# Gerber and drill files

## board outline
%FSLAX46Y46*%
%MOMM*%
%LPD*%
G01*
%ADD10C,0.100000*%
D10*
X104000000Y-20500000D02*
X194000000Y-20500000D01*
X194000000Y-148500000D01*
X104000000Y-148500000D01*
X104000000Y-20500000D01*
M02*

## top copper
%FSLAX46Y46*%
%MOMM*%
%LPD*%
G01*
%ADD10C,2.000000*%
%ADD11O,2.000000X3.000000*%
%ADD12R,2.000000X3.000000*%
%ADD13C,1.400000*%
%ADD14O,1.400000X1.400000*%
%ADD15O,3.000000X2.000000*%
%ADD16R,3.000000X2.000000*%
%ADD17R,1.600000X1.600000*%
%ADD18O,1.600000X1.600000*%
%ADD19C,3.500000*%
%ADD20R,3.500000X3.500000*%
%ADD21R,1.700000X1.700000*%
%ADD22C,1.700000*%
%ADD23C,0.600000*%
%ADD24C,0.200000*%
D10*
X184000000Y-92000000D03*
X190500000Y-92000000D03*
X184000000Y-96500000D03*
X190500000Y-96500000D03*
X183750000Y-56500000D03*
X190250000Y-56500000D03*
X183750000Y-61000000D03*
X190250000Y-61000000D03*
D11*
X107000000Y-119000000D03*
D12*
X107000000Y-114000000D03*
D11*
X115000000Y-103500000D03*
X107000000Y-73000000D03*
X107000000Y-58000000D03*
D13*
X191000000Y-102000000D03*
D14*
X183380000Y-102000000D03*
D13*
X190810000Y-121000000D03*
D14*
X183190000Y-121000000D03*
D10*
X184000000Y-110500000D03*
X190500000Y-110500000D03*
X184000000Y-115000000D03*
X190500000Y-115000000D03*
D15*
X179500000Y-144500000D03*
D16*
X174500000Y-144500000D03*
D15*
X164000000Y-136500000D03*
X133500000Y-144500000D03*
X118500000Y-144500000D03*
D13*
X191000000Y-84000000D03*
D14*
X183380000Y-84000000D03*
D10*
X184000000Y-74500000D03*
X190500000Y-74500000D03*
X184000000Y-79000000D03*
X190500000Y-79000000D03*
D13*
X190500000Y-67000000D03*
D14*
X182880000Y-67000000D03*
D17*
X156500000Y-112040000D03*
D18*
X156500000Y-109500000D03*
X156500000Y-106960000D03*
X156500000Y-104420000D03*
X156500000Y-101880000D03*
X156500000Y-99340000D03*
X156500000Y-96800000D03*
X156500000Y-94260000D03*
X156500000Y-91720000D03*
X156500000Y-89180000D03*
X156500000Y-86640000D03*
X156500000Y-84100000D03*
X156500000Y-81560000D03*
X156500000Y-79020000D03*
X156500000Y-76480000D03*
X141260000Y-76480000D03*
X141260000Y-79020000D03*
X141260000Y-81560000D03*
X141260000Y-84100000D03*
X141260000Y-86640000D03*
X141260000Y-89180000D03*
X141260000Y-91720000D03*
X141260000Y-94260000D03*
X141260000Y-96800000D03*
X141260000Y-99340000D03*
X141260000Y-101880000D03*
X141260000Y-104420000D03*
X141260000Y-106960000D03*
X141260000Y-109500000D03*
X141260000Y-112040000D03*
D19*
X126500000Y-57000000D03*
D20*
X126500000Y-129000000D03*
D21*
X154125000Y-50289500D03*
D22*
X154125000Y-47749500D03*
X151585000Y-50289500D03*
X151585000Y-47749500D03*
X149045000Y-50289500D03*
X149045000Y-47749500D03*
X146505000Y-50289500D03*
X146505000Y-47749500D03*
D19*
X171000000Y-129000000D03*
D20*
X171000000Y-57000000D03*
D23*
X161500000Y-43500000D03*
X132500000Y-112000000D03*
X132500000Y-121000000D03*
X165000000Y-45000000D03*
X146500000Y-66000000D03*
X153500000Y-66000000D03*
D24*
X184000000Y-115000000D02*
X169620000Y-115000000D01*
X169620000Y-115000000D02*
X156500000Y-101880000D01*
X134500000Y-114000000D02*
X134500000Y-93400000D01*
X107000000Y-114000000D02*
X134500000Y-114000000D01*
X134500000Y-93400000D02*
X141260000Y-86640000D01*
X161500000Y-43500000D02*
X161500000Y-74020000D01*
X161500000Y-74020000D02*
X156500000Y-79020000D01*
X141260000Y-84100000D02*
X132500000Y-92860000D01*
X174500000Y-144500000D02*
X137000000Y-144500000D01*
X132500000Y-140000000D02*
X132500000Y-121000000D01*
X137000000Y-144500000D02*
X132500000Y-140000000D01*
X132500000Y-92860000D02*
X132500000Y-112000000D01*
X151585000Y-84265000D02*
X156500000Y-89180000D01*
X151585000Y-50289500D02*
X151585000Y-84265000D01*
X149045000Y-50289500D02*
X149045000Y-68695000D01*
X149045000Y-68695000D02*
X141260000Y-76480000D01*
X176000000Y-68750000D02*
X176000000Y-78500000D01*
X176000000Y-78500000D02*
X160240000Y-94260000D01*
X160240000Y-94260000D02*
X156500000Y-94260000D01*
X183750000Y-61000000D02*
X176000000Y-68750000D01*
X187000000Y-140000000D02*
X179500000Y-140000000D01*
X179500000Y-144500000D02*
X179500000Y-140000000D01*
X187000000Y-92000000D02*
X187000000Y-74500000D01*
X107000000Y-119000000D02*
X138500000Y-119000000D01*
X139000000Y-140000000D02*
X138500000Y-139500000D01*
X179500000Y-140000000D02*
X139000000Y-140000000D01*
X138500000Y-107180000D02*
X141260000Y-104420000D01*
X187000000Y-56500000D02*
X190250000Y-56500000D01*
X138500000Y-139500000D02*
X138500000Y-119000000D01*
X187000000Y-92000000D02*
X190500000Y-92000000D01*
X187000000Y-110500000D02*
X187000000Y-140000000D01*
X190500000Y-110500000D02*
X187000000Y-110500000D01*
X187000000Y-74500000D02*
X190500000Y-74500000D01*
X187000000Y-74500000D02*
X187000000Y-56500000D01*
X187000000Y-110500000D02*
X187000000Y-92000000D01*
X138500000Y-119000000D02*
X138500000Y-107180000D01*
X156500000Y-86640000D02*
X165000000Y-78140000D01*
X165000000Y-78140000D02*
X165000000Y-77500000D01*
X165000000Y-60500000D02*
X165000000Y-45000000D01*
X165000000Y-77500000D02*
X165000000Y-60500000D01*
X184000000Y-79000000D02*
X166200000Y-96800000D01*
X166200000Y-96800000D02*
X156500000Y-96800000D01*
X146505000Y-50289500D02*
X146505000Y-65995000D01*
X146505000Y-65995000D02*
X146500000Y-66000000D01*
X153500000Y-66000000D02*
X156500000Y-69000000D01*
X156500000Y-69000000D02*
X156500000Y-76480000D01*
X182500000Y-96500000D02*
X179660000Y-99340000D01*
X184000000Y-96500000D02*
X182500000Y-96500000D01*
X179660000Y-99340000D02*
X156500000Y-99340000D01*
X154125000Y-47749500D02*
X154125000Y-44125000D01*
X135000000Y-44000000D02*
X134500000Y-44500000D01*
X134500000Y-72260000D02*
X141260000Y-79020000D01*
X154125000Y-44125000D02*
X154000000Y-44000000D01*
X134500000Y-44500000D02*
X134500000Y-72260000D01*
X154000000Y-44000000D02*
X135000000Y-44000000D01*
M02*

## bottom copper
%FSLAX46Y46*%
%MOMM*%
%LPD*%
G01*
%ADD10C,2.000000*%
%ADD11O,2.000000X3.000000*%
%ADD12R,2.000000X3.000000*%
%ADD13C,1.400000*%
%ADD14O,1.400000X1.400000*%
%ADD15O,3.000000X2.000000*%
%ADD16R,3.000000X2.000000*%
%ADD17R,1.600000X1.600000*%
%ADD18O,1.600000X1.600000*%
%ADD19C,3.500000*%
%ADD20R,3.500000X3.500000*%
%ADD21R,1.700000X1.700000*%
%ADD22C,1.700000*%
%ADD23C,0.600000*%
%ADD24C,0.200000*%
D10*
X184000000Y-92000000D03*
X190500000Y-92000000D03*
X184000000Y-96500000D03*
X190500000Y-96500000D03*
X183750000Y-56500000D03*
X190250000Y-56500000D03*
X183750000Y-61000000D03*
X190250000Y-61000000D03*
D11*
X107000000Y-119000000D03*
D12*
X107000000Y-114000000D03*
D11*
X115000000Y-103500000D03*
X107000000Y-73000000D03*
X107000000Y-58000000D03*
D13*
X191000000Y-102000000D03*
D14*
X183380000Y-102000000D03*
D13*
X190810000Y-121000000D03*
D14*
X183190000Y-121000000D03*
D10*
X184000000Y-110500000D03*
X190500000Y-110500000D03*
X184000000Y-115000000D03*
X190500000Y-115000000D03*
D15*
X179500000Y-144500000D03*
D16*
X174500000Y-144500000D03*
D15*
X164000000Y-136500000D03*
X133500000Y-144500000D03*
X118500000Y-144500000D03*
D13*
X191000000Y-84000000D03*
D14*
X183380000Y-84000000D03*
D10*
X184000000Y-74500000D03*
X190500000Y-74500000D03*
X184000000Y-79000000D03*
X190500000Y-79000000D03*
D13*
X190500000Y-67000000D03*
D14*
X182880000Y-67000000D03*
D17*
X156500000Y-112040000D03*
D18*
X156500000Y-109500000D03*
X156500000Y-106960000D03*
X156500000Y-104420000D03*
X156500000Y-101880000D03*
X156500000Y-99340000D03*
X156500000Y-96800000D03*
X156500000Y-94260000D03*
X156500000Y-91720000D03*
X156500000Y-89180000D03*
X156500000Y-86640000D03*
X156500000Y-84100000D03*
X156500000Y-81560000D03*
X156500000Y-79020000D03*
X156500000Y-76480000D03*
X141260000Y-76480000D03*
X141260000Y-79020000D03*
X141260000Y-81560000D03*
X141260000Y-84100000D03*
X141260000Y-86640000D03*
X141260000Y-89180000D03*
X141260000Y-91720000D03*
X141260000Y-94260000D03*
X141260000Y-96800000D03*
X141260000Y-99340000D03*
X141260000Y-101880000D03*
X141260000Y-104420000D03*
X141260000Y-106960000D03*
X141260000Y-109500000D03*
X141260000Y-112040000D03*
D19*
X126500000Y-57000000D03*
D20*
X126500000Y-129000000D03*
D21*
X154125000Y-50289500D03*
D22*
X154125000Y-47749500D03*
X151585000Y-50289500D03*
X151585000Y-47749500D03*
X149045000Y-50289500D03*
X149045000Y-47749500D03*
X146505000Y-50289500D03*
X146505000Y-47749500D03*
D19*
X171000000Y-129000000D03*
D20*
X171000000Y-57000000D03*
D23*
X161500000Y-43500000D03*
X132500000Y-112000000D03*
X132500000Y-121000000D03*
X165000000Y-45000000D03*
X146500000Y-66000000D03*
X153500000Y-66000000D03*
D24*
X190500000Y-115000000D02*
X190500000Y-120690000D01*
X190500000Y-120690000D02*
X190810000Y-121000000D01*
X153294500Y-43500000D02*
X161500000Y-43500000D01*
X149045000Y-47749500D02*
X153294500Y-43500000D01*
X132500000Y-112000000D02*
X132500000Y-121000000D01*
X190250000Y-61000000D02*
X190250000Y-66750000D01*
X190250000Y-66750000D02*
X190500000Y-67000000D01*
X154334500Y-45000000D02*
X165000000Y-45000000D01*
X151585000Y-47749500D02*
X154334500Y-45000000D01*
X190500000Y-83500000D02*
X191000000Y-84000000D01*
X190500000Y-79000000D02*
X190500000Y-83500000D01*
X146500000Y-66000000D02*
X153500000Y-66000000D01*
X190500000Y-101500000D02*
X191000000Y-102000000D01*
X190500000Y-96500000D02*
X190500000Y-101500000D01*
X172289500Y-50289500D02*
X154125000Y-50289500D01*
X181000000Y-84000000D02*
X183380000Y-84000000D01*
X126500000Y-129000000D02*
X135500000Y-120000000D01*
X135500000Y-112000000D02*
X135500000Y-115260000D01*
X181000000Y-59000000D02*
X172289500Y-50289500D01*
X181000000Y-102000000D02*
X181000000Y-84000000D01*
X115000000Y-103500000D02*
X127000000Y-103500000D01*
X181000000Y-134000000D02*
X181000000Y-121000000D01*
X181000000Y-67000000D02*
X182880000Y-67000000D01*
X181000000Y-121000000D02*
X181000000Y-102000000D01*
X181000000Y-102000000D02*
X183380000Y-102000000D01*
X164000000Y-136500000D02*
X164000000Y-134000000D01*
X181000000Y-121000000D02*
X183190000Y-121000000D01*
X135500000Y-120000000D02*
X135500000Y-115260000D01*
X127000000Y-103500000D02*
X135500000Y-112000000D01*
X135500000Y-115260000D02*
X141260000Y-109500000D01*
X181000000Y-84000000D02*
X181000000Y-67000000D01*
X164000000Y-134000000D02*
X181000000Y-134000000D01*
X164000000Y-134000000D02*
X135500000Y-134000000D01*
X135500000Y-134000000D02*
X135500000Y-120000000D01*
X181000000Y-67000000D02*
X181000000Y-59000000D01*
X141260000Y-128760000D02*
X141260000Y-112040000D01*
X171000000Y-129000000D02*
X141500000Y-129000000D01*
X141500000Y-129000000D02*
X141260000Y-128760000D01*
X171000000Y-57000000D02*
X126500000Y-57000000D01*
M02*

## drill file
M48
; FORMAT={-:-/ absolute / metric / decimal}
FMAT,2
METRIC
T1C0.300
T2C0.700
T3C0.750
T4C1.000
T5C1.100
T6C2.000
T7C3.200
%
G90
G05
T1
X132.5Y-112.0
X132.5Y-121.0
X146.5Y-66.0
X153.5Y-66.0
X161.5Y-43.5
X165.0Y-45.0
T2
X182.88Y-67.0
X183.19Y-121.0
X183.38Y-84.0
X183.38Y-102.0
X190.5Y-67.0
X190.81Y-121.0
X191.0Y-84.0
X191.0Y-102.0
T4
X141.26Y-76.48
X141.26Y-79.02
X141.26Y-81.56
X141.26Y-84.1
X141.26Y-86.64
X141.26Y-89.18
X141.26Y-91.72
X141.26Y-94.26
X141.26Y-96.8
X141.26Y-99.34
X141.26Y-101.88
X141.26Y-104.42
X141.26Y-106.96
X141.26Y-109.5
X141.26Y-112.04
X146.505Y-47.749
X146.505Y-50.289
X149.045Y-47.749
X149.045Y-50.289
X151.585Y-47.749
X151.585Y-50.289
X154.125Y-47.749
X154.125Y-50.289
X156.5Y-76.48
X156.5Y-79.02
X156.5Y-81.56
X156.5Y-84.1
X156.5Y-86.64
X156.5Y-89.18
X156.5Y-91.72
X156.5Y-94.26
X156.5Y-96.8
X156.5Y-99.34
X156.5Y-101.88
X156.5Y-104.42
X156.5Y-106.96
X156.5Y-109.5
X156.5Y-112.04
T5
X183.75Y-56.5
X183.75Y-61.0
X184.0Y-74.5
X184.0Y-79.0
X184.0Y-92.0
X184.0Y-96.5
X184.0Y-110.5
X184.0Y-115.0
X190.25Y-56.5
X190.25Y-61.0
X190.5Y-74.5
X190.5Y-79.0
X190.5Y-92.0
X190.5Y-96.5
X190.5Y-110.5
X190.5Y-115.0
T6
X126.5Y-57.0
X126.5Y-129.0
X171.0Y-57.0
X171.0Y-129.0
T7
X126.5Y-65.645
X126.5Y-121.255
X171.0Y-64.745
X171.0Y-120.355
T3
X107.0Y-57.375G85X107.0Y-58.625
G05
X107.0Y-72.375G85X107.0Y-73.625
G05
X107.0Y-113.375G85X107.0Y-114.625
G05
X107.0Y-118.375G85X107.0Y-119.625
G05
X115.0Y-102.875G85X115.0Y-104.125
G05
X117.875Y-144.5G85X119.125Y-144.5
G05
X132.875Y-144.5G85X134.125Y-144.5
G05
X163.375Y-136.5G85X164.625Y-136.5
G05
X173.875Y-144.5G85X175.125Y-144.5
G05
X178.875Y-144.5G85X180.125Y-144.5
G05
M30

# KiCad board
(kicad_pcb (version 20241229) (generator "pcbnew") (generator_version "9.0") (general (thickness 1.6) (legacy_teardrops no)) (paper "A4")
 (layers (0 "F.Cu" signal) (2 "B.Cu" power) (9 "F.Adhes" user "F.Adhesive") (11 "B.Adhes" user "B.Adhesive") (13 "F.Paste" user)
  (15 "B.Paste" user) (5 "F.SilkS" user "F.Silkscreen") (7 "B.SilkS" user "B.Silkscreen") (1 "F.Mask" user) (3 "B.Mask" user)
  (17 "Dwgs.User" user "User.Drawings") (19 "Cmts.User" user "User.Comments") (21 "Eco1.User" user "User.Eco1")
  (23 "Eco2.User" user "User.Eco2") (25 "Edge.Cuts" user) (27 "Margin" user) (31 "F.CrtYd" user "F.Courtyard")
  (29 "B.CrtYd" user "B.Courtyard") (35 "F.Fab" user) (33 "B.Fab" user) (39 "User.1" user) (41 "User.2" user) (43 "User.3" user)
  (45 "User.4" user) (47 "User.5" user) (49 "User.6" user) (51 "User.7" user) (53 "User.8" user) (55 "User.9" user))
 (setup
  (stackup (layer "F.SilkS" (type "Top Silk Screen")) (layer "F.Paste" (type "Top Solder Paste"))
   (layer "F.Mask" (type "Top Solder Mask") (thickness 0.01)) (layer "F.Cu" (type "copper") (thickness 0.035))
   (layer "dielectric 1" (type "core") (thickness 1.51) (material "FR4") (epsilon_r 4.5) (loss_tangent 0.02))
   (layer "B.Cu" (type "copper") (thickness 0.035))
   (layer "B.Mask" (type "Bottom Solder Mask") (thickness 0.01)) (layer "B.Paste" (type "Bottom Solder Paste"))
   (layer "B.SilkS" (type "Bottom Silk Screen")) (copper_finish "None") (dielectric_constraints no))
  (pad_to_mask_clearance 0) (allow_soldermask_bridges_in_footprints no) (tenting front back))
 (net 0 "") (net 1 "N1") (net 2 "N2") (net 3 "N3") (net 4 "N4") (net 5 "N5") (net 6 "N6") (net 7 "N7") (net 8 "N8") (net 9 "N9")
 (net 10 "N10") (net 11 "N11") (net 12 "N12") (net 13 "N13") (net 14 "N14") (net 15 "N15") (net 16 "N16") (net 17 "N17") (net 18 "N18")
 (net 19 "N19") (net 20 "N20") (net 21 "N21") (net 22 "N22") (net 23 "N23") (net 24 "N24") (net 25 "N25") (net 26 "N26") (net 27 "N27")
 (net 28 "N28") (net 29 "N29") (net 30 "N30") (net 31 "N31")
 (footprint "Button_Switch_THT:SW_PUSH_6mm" (layer "F.Cu") (at 184 92)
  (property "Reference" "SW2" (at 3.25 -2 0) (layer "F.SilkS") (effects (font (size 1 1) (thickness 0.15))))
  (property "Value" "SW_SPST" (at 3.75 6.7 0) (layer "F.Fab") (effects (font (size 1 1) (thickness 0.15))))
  (pad "1" thru_hole circle (at 0 0 90) (size 2 2) (drill 1.1) (layers "*.Cu" "*.Mask") (remove_unused_layers no) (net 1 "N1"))
  (pad "1" thru_hole circle (at 6.5 0 90) (size 2 2) (drill 1.1) (layers "*.Cu" "*.Mask") (remove_unused_layers no) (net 1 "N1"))
  (pad "2" thru_hole circle (at 0 4.5 90) (size 2 2) (drill 1.1) (layers "*.Cu" "*.Mask") (remove_unused_layers no) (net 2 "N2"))
  (pad "2" thru_hole circle (at 6.5 4.5 90) (size 2 2) (drill 1.1) (layers "*.Cu" "*.Mask") (remove_unused_layers no) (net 2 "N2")))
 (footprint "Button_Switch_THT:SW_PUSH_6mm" (layer "F.Cu") (at 183.75 56.5)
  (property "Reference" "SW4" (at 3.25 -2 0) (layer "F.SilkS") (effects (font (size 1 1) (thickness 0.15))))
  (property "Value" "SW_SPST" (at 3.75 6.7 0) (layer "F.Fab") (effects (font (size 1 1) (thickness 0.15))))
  (pad "1" thru_hole circle (at 0 0 90) (size 2 2) (drill 1.1) (layers "*.Cu" "*.Mask") (remove_unused_layers no) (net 1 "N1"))
  (pad "1" thru_hole circle (at 6.5 0 90) (size 2 2) (drill 1.1) (layers "*.Cu" "*.Mask") (remove_unused_layers no) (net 1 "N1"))
  (pad "2" thru_hole circle (at 0 4.5 90) (size 2 2) (drill 1.1) (layers "*.Cu" "*.Mask") (remove_unused_layers no) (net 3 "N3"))
  (pad "2" thru_hole circle (at 6.5 4.5 90) (size 2 2) (drill 1.1) (layers "*.Cu" "*.Mask") (remove_unused_layers no) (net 3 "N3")))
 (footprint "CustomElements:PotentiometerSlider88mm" (layer "F.Cu") (at 111 88.5 -90)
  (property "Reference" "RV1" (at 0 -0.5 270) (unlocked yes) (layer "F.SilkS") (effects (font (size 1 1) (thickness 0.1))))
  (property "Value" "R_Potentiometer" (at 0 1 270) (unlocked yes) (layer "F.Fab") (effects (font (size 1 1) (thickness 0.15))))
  (pad "1" thru_hole oval (at 30.5 4 270) (size 3 2) (drill oval 2 0.75) (layers "*.Cu" "*.Mask") (remove_unused_layers no) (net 1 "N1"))
  (pad "2" thru_hole rect (at 25.5 4 270) (size 3 2) (drill oval 2 0.75) (layers "*.Cu" "*.Mask") (remove_unused_layers no) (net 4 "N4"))
  (pad "3" thru_hole oval (at 15 -4 270) (size 3 2) (drill oval 2 0.75) (layers "*.Cu" "*.Mask") (remove_unused_layers no) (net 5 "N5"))
  (pad "4" thru_hole oval (at -15.5 4 270) (size 3 2) (drill oval 2 0.75) (layers "*.Cu" "*.Mask") (remove_unused_layers no))
  (pad "5" thru_hole oval (at -30.5 4 270) (size 3 2) (drill oval 2 0.75) (layers "*.Cu" "*.Mask") (remove_unused_layers no)))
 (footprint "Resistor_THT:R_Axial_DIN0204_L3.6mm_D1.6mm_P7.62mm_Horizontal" (layer "F.Cu") (at 191 102 180)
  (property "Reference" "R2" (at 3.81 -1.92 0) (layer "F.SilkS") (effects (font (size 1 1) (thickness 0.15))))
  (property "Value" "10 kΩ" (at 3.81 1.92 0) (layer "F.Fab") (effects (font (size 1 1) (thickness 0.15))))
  (pad "1" thru_hole circle (at 0 0 180) (size 1.4 1.4) (drill 0.7) (layers "*.Cu" "*.Mask") (remove_unused_layers no) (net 2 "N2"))
  (pad "2" thru_hole oval (at 7.62 0 180) (size 1.4 1.4) (drill 0.7) (layers "*.Cu" "*.Mask") (remove_unused_layers no) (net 5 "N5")))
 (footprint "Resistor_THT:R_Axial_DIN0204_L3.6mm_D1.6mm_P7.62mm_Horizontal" (layer "F.Cu") (at 190.81 121 180)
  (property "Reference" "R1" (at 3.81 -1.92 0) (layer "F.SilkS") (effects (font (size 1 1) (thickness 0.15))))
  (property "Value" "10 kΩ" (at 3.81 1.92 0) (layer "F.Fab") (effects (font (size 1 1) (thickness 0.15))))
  (pad "1" thru_hole circle (at 0 0 180) (size 1.4 1.4) (drill 0.7) (layers "*.Cu" "*.Mask") (remove_unused_layers no) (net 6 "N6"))
  (pad "2" thru_hole oval (at 7.62 0 180) (size 1.4 1.4) (drill 0.7) (layers "*.Cu" "*.Mask") (remove_unused_layers no) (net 5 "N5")))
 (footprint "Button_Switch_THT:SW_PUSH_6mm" (layer "F.Cu") (at 184 110.5)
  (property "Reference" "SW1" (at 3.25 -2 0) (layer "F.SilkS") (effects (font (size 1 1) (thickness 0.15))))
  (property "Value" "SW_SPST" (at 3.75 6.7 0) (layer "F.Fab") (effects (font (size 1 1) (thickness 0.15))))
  (pad "1" thru_hole circle (at 0 0 90) (size 2 2) (drill 1.1) (layers "*.Cu" "*.Mask") (remove_unused_layers no) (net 1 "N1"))
  (pad "1" thru_hole circle (at 6.5 0 90) (size 2 2) (drill 1.1) (layers "*.Cu" "*.Mask") (remove_unused_layers no) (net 1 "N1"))
  (pad "2" thru_hole circle (at 0 4.5 90) (size 2 2) (drill 1.1) (layers "*.Cu" "*.Mask") (remove_unused_layers no) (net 6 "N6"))
  (pad "2" thru_hole circle (at 6.5 4.5 90) (size 2 2) (drill 1.1) (layers "*.Cu" "*.Mask") (remove_unused_layers no) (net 6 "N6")))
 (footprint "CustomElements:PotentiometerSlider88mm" (layer "F.Cu") (at 149 140.5)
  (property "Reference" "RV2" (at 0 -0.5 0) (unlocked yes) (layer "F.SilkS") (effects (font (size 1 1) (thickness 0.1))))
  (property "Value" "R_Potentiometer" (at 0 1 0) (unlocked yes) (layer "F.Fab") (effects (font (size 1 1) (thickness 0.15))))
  (pad "1" thru_hole oval (at 30.5 4) (size 3 2) (drill oval 2 0.75) (layers "*.Cu" "*.Mask") (remove_unused_layers no) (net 1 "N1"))
  (pad "2" thru_hole rect (at 25.5 4) (size 3 2) (drill oval 2 0.75) (layers "*.Cu" "*.Mask") (remove_unused_layers no) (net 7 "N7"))
  (pad "3" thru_hole oval (at 15 -4) (size 3 2) (drill oval 2 0.75) (layers "*.Cu" "*.Mask") (remove_unused_layers no) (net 5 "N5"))
  (pad "4" thru_hole oval (at -15.5 4) (size 3 2) (drill oval 2 0.75) (layers "*.Cu" "*.Mask") (remove_unused_layers no))
  (pad "5" thru_hole oval (at -30.5 4) (size 3 2) (drill oval 2 0.75) (layers "*.Cu" "*.Mask") (remove_unused_layers no)))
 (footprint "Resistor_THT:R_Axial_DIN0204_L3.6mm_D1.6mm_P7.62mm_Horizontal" (layer "F.Cu") (at 191 84 180)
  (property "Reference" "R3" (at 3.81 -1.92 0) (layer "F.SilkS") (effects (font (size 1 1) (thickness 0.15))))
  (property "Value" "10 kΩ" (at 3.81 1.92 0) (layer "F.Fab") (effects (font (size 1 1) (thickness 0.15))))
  (pad "1" thru_hole circle (at 0 0 180) (size 1.4 1.4) (drill 0.7) (layers "*.Cu" "*.Mask") (remove_unused_layers no) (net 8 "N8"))
  (pad "2" thru_hole oval (at 7.62 0 180) (size 1.4 1.4) (drill 0.7) (layers "*.Cu" "*.Mask") (remove_unused_layers no) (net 5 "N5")))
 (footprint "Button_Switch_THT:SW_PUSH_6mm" (layer "F.Cu") (at 184 74.5)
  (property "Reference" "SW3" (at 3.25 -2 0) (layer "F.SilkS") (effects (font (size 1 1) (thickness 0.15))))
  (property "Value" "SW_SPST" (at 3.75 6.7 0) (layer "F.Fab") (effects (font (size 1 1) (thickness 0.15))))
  (pad "1" thru_hole circle (at 0 0 90) (size 2 2) (drill 1.1) (layers "*.Cu" "*.Mask") (remove_unused_layers no) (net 1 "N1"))
  (pad "1" thru_hole circle (at 6.5 0 90) (size 2 2) (drill 1.1) (layers "*.Cu" "*.Mask") (remove_unused_layers no) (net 1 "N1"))
  (pad "2" thru_hole circle (at 0 4.5 90) (size 2 2) (drill 1.1) (layers "*.Cu" "*.Mask") (remove_unused_layers no) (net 8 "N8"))
  (pad "2" thru_hole circle (at 6.5 4.5 90) (size 2 2) (drill 1.1) (layers "*.Cu" "*.Mask") (remove_unused_layers no) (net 8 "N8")))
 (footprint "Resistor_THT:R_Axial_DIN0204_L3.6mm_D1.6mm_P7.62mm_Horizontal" (layer "F.Cu") (at 190.5 67 180)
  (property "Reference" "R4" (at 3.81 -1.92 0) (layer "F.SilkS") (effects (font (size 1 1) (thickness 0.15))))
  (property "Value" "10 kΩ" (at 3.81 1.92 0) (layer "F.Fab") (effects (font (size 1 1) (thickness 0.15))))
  (pad "1" thru_hole circle (at 0 0 180) (size 1.4 1.4) (drill 0.7) (layers "*.Cu" "*.Mask") (remove_unused_layers no) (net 3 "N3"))
  (pad "2" thru_hole oval (at 7.62 0 180) (size 1.4 1.4) (drill 0.7) (layers "*.Cu" "*.Mask") (remove_unused_layers no) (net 5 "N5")))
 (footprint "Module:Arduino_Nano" (layer "F.Cu") (at 156.5 112.04 180)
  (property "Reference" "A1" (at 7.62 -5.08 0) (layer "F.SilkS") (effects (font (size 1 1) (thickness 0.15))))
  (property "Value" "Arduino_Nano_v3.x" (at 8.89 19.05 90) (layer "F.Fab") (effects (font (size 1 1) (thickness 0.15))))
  (pad "1" thru_hole rect (at 0 0 180) (size 1.6 1.6) (drill 1) (layers "*.Cu" "*.Mask") (remove_unused_layers no) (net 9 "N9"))
  (pad "2" thru_hole oval (at 0 2.54 180) (size 1.6 1.6) (drill 1) (layers "*.Cu" "*.Mask") (remove_unused_layers no) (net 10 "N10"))
  (pad "3" thru_hole oval (at 0 5.08 180) (size 1.6 1.6) (drill 1) (layers "*.Cu" "*.Mask") (remove_unused_layers no) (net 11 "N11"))
  (pad "4" thru_hole oval (at 0 7.62 180) (size 1.6 1.6) (drill 1) (layers "*.Cu" "*.Mask") (remove_unused_layers no) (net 5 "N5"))
  (pad "5" thru_hole oval (at 0 10.16 180) (size 1.6 1.6) (drill 1) (layers "*.Cu" "*.Mask") (remove_unused_layers no) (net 6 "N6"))
  (pad "6" thru_hole oval (at 0 12.7 180) (size 1.6 1.6) (drill 1) (layers "*.Cu" "*.Mask") (remove_unused_layers no) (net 2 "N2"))
  (pad "7" thru_hole oval (at 0 15.24 180) (size 1.6 1.6) (drill 1) (layers "*.Cu" "*.Mask") (remove_unused_layers no) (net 8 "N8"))
  (pad "8" thru_hole oval (at 0 17.78 180) (size 1.6 1.6) (drill 1) (layers "*.Cu" "*.Mask") (remove_unused_layers no) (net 3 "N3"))
  (pad "9" thru_hole oval (at 0 20.32 180) (size 1.6 1.6) (drill 1) (layers "*.Cu" "*.Mask") (remove_unused_layers no) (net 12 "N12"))
  (pad "10" thru_hole oval (at 0 22.86 180) (size 1.6 1.6) (drill 1) (layers "*.Cu" "*.Mask") (remove_unused_layers no) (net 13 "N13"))
  (pad "11" thru_hole oval (at 0 25.4 180) (size 1.6 1.6) (drill 1) (layers "*.Cu" "*.Mask") (remove_unused_layers no) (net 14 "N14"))
  (pad "12" thru_hole oval (at 0 27.94 180) (size 1.6 1.6) (drill 1) (layers "*.Cu" "*.Mask") (remove_unused_layers no) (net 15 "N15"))
  (pad "13" thru_hole oval (at 0 30.48 180) (size 1.6 1.6) (drill 1) (layers "*.Cu" "*.Mask") (remove_unused_layers no) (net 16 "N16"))
  (pad "14" thru_hole oval (at 0 33.02 180) (size 1.6 1.6) (drill 1) (layers "*.Cu" "*.Mask") (remove_unused_layers no) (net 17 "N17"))
  (pad "15" thru_hole oval (at 0 35.56 180) (size 1.6 1.6) (drill 1) (layers "*.Cu" "*.Mask") (remove_unused_layers no) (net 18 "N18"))
  (pad "16" thru_hole oval (at 15.24 35.56 180) (size 1.6 1.6) (drill 1) (layers "*.Cu" "*.Mask") (remove_unused_layers no) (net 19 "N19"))
  (pad "17" thru_hole oval (at 15.24 33.02 180) (size 1.6 1.6) (drill 1) (layers "*.Cu" "*.Mask") (remove_unused_layers no) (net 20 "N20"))
  (pad "18" thru_hole oval (at 15.24 30.48 180) (size 1.6 1.6) (drill 1) (layers "*.Cu" "*.Mask") (remove_unused_layers no) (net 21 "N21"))
  (pad "19" thru_hole oval (at 15.24 27.94 180) (size 1.6 1.6) (drill 1) (layers "*.Cu" "*.Mask") (remove_unused_layers no) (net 7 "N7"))
  (pad "20" thru_hole oval (at 15.24 25.4 180) (size 1.6 1.6) (drill 1) (layers "*.Cu" "*.Mask") (remove_unused_layers no) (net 4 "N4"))
  (pad "21" thru_hole oval (at 15.24 22.86 180) (size 1.6 1.6) (drill 1) (layers "*.Cu" "*.Mask") (remove_unused_layers no) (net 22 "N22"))
  (pad "22" thru_hole oval (at 15.24 20.32 180) (size 1.6 1.6) (drill 1) (layers "*.Cu" "*.Mask") (remove_unused_layers no) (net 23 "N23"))
  (pad "23" thru_hole oval (at 15.24 17.78 180) (size 1.6 1.6) (drill 1) (layers "*.Cu" "*.Mask") (remove_unused_layers no) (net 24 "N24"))
  (pad "24" thru_hole oval (at 15.24 15.24 180) (size 1.6 1.6) (drill 1) (layers "*.Cu" "*.Mask") (remove_unused_layers no) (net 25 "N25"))
  (pad "25" thru_hole oval (at 15.24 12.7 180) (size 1.6 1.6) (drill 1) (layers "*.Cu" "*.Mask") (remove_unused_layers no) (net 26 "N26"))
  (pad "26" thru_hole oval (at 15.24 10.16 180) (size 1.6 1.6) (drill 1) (layers "*.Cu" "*.Mask") (remove_unused_layers no) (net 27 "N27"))
  (pad "27" thru_hole oval (at 15.24 7.62 180) (size 1.6 1.6) (drill 1) (layers "*.Cu" "*.Mask") (remove_unused_layers no) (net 1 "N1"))
  (pad "28" thru_hole oval (at 15.24 5.08 180) (size 1.6 1.6) (drill 1) (layers "*.Cu" "*.Mask") (remove_unused_layers no) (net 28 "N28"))
  (pad "29" thru_hole oval (at 15.24 2.54 180) (size 1.6 1.6) (drill 1) (layers "*.Cu" "*.Mask") (remove_unused_layers no) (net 5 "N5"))
  (pad "30" thru_hole oval (at 15.24 0 180) (size 1.6 1.6) (drill 1) (layers "*.Cu" "*.Mask") (remove_unused_layers no) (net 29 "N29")))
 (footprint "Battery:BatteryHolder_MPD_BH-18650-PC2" (layer "B.Cu") (at 126.5 57 -90)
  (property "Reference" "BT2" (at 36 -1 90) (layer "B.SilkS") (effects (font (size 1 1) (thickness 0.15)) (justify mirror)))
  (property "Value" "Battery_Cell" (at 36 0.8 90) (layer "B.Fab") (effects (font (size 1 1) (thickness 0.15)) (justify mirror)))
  (pad "" np_thru_hole circle (at 8.645 0 270) (size 3.2 3.2) (drill 3.2) (layers "*.Cu" "*.Mask"))
  (pad "" np_thru_hole circle (at 64.255 0 270) (size 3.2 3.2) (drill 3.2) (layers "*.Cu" "*.Mask"))
  (pad "1" thru_hole circle (at 0 0 270) (size 3.5 3.5) (drill 2) (layers "*.Cu" "*.Mask") (remove_unused_layers no) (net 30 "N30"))
  (pad "2" thru_hole rect (at 72 0 270) (size 3.5 3.5) (drill 2) (layers "*.Cu" "*.Mask") (remove_unused_layers no) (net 5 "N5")))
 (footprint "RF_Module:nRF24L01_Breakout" (layer "B.Cu") (at 154.125 50.2895 90)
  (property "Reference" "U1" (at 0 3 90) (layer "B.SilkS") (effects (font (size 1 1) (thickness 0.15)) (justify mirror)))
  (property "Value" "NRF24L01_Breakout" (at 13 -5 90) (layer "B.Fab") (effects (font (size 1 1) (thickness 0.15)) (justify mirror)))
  (pad "1" thru_hole rect (at 0 0 90) (size 1.7 1.7) (drill 1) (layers "*.Cu" "*.Mask") (remove_unused_layers no) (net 5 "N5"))
  (pad "2" thru_hole circle (at 2.54 0 90) (size 1.7 1.7) (drill 1) (layers "*.Cu" "*.Mask") (remove_unused_layers no) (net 20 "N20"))
  (pad "3" thru_hole circle (at 0 -2.54 90) (size 1.7 1.7) (drill 1) (layers "*.Cu" "*.Mask") (remove_unused_layers no) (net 13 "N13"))
  (pad "4" thru_hole circle (at 2.54 -2.54 90) (size 1.7 1.7) (drill 1) (layers "*.Cu" "*.Mask") (remove_unused_layers no) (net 14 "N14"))
  (pad "5" thru_hole circle (at 0 -5.08 90) (size 1.7 1.7) (drill 1) (layers "*.Cu" "*.Mask") (remove_unused_layers no) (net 19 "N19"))
  (pad "6" thru_hole circle (at 2.54 -5.08 90) (size 1.7 1.7) (drill 1) (layers "*.Cu" "*.Mask") (remove_unused_layers no) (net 17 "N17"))
  (pad "7" thru_hole circle (at 0 -7.62 90) (size 1.7 1.7) (drill 1) (layers "*.Cu" "*.Mask") (remove_unused_layers no) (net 18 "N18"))
  (pad "8" thru_hole circle (at 2.54 -7.62 90) (size 1.7 1.7) (drill 1) (layers "*.Cu" "*.Mask") (remove_unused_layers no) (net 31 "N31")))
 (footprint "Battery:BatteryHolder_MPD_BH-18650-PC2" (layer "B.Cu") (at 171 129 90)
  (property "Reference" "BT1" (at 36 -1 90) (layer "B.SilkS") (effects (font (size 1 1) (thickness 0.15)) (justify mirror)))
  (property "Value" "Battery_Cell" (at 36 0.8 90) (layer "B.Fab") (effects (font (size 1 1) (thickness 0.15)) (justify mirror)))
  (pad "" np_thru_hole circle (at 8.645 0 90) (size 3.2 3.2) (drill 3.2) (layers "*.Cu" "*.Mask"))
  (pad "" np_thru_hole circle (at 64.255 0 90) (size 3.2 3.2) (drill 3.2) (layers "*.Cu" "*.Mask"))
  (pad "1" thru_hole circle (at 0 0 90) (size 3.5 3.5) (drill 2) (layers "*.Cu" "*.Mask") (remove_unused_layers no) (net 29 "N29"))
  (pad "2" thru_hole rect (at 72 0 90) (size 3.5 3.5) (drill 2) (layers "*.Cu" "*.Mask") (remove_unused_layers no) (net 30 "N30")))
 (gr_rect (start 104 20.5) (end 194 148.5) (stroke (width 0.1) (type default)) (fill no) (layer "Edge.Cuts"))
 (segment (start 184 115) (end 169.62 115) (width 0.2) (layer "F.Cu") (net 6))
 (segment (start 169.62 115) (end 156.5 101.88) (width 0.2) (layer "F.Cu") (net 6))
 (segment (start 190.5 115) (end 190.5 120.69) (width 0.2) (layer "B.Cu") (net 6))
 (segment (start 190.5 120.69) (end 190.81 121) (width 0.2) (layer "B.Cu") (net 6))
 (segment (start 134.5 114) (end 134.5 93.4) (width 0.2) (layer "F.Cu") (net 4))
 (segment (start 107 114) (end 134.5 114) (width 0.2) (layer "F.Cu") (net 4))
 (segment (start 134.5 93.4) (end 141.26 86.64) (width 0.2) (layer "F.Cu") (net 4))
 (segment (start 161.5 43.5) (end 161.5 74.02) (width 0.2) (layer "F.Cu") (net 17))
 (segment (start 161.5 74.02) (end 156.5 79.02) (width 0.2) (layer "F.Cu") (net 17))
 (via (at 161.5 43.5) (size 0.6) (drill 0.3) (layers "F.Cu" "B.Cu") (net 17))
 (segment (start 153.2945 43.5) (end 161.5 43.5) (width 0.2) (layer "B.Cu") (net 17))
 (segment (start 149.045 47.7495) (end 153.2945 43.5) (width 0.2) (layer "B.Cu") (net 17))
 (segment (start 141.26 84.1) (end 132.5 92.86) (width 0.2) (layer "F.Cu") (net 7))
 (segment (start 174.5 144.5) (end 137 144.5) (width 0.2) (layer "F.Cu") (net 7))
 (segment (start 132.5 140) (end 132.5 121) (width 0.2) (layer "F.Cu") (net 7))
 (segment (start 137 144.5) (end 132.5 140) (width 0.2) (layer "F.Cu") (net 7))
 (segment (start 132.5 92.86) (end 132.5 112) (width 0.2) (layer "F.Cu") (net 7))
 (via (at 132.5 112) (size 0.6) (drill 0.3) (layers "F.Cu" "B.Cu") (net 7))
 (via (at 132.5 121) (size 0.6) (drill 0.3) (layers "F.Cu" "B.Cu") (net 7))
 (segment (start 132.5 112) (end 132.5 121) (width 0.2) (layer "B.Cu") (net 7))
 (segment (start 151.585 84.265) (end 156.5 89.18) (width 0.2) (layer "F.Cu") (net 13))
 (segment (start 151.585 50.2895) (end 151.585 84.265) (width 0.2) (layer "F.Cu") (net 13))
 (segment (start 149.045 50.2895) (end 149.045 68.695) (width 0.2) (layer "F.Cu") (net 19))
 (segment (start 149.045 68.695) (end 141.26 76.48) (width 0.2) (layer "F.Cu") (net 19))
 (segment (start 176 68.75) (end 176 78.5) (width 0.2) (layer "F.Cu") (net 3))
 (segment (start 176 78.5) (end 160.24 94.26) (width 0.2) (layer "F.Cu") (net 3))
 (segment (start 160.24 94.26) (end 156.5 94.26) (width 0.2) (layer "F.Cu") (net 3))
 (segment (start 183.75 61) (end 176 68.75) (width 0.2) (layer "F.Cu") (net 3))
 (segment (start 190.25 61) (end 190.25 66.75) (width 0.2) (layer "B.Cu") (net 3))
 (segment (start 190.25 66.75) (end 190.5 67) (width 0.2) (layer "B.Cu") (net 3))
 (segment (start 187 140) (end 179.5 140) (width 0.2) (layer "F.Cu") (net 1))
 (segment (start 179.5 144.5) (end 179.5 140) (width 0.2) (layer "F.Cu") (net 1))
 (segment (start 187 92) (end 187 74.5) (width 0.2) (layer "F.Cu") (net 1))
 (segment (start 107 119) (end 138.5 119) (width 0.2) (layer "F.Cu") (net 1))
 (segment (start 139 140) (end 138.5 139.5) (width 0.2) (layer "F.Cu") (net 1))
 (segment (start 179.5 140) (end 139 140) (width 0.2) (layer "F.Cu") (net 1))
 (segment (start 138.5 107.18) (end 141.26 104.42) (width 0.2) (layer "F.Cu") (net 1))
 (segment (start 187 56.5) (end 190.25 56.5) (width 0.2) (layer "F.Cu") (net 1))
 (segment (start 138.5 139.5) (end 138.5 119) (width 0.2) (layer "F.Cu") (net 1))
 (segment (start 187 92) (end 190.5 92) (width 0.2) (layer "F.Cu") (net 1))
 (segment (start 187 110.5) (end 187 140) (width 0.2) (layer "F.Cu") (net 1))
 (segment (start 190.5 110.5) (end 187 110.5) (width 0.2) (layer "F.Cu") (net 1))
 (segment (start 187 74.5) (end 190.5 74.5) (width 0.2) (layer "F.Cu") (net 1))
 (segment (start 187 74.5) (end 187 56.5) (width 0.2) (layer "F.Cu") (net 1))
 (segment (start 187 110.5) (end 187 92) (width 0.2) (layer "F.Cu") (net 1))
 (segment (start 138.5 119) (end 138.5 107.18) (width 0.2) (layer "F.Cu") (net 1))
 (segment (start 156.5 86.64) (end 165 78.14) (width 0.2) (layer "F.Cu") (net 14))
 (segment (start 165 78.14) (end 165 77.5) (width 0.2) (layer "F.Cu") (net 14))
 (segment (start 165 60.5) (end 165 45) (width 0.2) (layer "F.Cu") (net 14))
 (segment (start 165 77.5) (end 165 60.5) (width 0.2) (layer "F.Cu") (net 14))
 (via (at 165 45) (size 0.6) (drill 0.3) (layers "F.Cu" "B.Cu") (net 14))
 (segment (start 154.3345 45) (end 165 45) (width 0.2) (layer "B.Cu") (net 14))
 (segment (start 151.585 47.7495) (end 154.3345 45) (width 0.2) (layer "B.Cu") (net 14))
 (segment (start 184 79) (end 166.2 96.8) (width 0.2) (layer "F.Cu") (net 8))
 (segment (start 166.2 96.8) (end 156.5 96.8) (width 0.2) (layer "F.Cu") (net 8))
 (segment (start 190.5 83.5) (end 191 84) (width 0.2) (layer "B.Cu") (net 8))
 (segment (start 190.5 79) (end 190.5 83.5) (width 0.2) (layer "B.Cu") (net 8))
 (segment (start 146.505 50.2895) (end 146.505 65.995) (width 0.2) (layer "F.Cu") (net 18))
 (segment (start 146.505 65.995) (end 146.5 66) (width 0.2) (layer "F.Cu") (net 18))
 (segment (start 153.5 66) (end 156.5 69) (width 0.2) (layer "F.Cu") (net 18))
 (segment (start 156.5 69) (end 156.5 76.48) (width 0.2) (layer "F.Cu") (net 18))
 (via (at 146.5 66) (size 0.6) (drill 0.3) (layers "F.Cu" "B.Cu") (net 18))
 (via (at 153.5 66) (size 0.6) (drill 0.3) (layers "F.Cu" "B.Cu") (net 18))
 (segment (start 146.5 66) (end 153.5 66) (width 0.2) (layer "B.Cu") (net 18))
 (segment (start 182.5 96.5) (end 179.66 99.34) (width 0.2) (layer "F.Cu") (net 2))
 (segment (start 184 96.5) (end 182.5 96.5) (width 0.2) (layer "F.Cu") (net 2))
 (segment (start 179.66 99.34) (end 156.5 99.34) (width 0.2) (layer "F.Cu") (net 2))
 (segment (start 190.5 101.5) (end 191 102) (width 0.2) (layer "B.Cu") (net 2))
 (segment (start 190.5 96.5) (end 190.5 101.5) (width 0.2) (layer "B.Cu") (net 2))
 (segment (start 154.125 47.7495) (end 154.125 44.125) (width 0.2) (layer "F.Cu") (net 20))
 (segment (start 135 44) (end 134.5 44.5) (width 0.2) (layer "F.Cu") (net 20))
 (segment (start 134.5 72.26) (end 141.26 79.02) (width 0.2) (layer "F.Cu") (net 20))
 (segment (start 154.125 44.125) (end 154 44) (width 0.2) (layer "F.Cu") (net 20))
 (segment (start 134.5 44.5) (end 134.5 72.26) (width 0.2) (layer "F.Cu") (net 20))
 (segment (start 154 44) (end 135 44) (width 0.2) (layer "F.Cu") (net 20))
 (segment (start 172.2895 50.2895) (end 154.125 50.2895) (width 0.2) (layer "B.Cu") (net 5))
 (segment (start 181 84) (end 183.38 84) (width 0.2) (layer "B.Cu") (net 5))
 (segment (start 126.5 129) (end 135.5 120) (width 0.2) (layer "B.Cu") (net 5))
 (segment (start 135.5 112) (end 135.5 115.26) (width 0.2) (layer "B.Cu") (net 5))
 (segment (start 181 59) (end 172.2895 50.2895) (width 0.2) (layer "B.Cu") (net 5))
 (segment (start 181 102) (end 181 84) (width 0.2) (layer "B.Cu") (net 5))
 (segment (start 115 103.5) (end 127 103.5) (width 0.2) (layer "B.Cu") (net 5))
 (segment (start 181 134) (end 181 121) (width 0.2) (layer "B.Cu") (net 5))
 (segment (start 181 67) (end 182.88 67) (width 0.2) (layer "B.Cu") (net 5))
 (segment (start 181 121) (end 181 102) (width 0.2) (layer "B.Cu") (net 5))
 (segment (start 181 102) (end 183.38 102) (width 0.2) (layer "B.Cu") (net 5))
 (segment (start 164 136.5) (end 164 134) (width 0.2) (layer "B.Cu") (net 5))
 (segment (start 181 121) (end 183.19 121) (width 0.2) (layer "B.Cu") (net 5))
 (segment (start 135.5 120) (end 135.5 115.26) (width 0.2) (layer "B.Cu") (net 5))
 (segment (start 127 103.5) (end 135.5 112) (width 0.2) (layer "B.Cu") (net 5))
 (segment (start 135.5 115.26) (end 141.26 109.5) (width 0.2) (layer "B.Cu") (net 5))
 (segment (start 181 84) (end 181 67) (width 0.2) (layer "B.Cu") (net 5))
 (segment (start 164 134) (end 181 134) (width 0.2) (layer "B.Cu") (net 5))
 (segment (start 164 134) (end 135.5 134) (width 0.2) (layer "B.Cu") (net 5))
 (segment (start 135.5 134) (end 135.5 120) (width 0.2) (layer "B.Cu") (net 5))
 (segment (start 181 67) (end 181 59) (width 0.2) (layer "B.Cu") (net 5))
 (segment (start 141.26 128.76) (end 141.26 112.04) (width 0.2) (layer "B.Cu") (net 29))
 (segment (start 171 129) (end 141.5 129) (width 0.2) (layer "B.Cu") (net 29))
 (segment (start 141.5 129) (end 141.26 128.76) (width 0.2) (layer "B.Cu") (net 29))
 (segment (start 171 57) (end 126.5 57) (width 0.2) (layer "B.Cu") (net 30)))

